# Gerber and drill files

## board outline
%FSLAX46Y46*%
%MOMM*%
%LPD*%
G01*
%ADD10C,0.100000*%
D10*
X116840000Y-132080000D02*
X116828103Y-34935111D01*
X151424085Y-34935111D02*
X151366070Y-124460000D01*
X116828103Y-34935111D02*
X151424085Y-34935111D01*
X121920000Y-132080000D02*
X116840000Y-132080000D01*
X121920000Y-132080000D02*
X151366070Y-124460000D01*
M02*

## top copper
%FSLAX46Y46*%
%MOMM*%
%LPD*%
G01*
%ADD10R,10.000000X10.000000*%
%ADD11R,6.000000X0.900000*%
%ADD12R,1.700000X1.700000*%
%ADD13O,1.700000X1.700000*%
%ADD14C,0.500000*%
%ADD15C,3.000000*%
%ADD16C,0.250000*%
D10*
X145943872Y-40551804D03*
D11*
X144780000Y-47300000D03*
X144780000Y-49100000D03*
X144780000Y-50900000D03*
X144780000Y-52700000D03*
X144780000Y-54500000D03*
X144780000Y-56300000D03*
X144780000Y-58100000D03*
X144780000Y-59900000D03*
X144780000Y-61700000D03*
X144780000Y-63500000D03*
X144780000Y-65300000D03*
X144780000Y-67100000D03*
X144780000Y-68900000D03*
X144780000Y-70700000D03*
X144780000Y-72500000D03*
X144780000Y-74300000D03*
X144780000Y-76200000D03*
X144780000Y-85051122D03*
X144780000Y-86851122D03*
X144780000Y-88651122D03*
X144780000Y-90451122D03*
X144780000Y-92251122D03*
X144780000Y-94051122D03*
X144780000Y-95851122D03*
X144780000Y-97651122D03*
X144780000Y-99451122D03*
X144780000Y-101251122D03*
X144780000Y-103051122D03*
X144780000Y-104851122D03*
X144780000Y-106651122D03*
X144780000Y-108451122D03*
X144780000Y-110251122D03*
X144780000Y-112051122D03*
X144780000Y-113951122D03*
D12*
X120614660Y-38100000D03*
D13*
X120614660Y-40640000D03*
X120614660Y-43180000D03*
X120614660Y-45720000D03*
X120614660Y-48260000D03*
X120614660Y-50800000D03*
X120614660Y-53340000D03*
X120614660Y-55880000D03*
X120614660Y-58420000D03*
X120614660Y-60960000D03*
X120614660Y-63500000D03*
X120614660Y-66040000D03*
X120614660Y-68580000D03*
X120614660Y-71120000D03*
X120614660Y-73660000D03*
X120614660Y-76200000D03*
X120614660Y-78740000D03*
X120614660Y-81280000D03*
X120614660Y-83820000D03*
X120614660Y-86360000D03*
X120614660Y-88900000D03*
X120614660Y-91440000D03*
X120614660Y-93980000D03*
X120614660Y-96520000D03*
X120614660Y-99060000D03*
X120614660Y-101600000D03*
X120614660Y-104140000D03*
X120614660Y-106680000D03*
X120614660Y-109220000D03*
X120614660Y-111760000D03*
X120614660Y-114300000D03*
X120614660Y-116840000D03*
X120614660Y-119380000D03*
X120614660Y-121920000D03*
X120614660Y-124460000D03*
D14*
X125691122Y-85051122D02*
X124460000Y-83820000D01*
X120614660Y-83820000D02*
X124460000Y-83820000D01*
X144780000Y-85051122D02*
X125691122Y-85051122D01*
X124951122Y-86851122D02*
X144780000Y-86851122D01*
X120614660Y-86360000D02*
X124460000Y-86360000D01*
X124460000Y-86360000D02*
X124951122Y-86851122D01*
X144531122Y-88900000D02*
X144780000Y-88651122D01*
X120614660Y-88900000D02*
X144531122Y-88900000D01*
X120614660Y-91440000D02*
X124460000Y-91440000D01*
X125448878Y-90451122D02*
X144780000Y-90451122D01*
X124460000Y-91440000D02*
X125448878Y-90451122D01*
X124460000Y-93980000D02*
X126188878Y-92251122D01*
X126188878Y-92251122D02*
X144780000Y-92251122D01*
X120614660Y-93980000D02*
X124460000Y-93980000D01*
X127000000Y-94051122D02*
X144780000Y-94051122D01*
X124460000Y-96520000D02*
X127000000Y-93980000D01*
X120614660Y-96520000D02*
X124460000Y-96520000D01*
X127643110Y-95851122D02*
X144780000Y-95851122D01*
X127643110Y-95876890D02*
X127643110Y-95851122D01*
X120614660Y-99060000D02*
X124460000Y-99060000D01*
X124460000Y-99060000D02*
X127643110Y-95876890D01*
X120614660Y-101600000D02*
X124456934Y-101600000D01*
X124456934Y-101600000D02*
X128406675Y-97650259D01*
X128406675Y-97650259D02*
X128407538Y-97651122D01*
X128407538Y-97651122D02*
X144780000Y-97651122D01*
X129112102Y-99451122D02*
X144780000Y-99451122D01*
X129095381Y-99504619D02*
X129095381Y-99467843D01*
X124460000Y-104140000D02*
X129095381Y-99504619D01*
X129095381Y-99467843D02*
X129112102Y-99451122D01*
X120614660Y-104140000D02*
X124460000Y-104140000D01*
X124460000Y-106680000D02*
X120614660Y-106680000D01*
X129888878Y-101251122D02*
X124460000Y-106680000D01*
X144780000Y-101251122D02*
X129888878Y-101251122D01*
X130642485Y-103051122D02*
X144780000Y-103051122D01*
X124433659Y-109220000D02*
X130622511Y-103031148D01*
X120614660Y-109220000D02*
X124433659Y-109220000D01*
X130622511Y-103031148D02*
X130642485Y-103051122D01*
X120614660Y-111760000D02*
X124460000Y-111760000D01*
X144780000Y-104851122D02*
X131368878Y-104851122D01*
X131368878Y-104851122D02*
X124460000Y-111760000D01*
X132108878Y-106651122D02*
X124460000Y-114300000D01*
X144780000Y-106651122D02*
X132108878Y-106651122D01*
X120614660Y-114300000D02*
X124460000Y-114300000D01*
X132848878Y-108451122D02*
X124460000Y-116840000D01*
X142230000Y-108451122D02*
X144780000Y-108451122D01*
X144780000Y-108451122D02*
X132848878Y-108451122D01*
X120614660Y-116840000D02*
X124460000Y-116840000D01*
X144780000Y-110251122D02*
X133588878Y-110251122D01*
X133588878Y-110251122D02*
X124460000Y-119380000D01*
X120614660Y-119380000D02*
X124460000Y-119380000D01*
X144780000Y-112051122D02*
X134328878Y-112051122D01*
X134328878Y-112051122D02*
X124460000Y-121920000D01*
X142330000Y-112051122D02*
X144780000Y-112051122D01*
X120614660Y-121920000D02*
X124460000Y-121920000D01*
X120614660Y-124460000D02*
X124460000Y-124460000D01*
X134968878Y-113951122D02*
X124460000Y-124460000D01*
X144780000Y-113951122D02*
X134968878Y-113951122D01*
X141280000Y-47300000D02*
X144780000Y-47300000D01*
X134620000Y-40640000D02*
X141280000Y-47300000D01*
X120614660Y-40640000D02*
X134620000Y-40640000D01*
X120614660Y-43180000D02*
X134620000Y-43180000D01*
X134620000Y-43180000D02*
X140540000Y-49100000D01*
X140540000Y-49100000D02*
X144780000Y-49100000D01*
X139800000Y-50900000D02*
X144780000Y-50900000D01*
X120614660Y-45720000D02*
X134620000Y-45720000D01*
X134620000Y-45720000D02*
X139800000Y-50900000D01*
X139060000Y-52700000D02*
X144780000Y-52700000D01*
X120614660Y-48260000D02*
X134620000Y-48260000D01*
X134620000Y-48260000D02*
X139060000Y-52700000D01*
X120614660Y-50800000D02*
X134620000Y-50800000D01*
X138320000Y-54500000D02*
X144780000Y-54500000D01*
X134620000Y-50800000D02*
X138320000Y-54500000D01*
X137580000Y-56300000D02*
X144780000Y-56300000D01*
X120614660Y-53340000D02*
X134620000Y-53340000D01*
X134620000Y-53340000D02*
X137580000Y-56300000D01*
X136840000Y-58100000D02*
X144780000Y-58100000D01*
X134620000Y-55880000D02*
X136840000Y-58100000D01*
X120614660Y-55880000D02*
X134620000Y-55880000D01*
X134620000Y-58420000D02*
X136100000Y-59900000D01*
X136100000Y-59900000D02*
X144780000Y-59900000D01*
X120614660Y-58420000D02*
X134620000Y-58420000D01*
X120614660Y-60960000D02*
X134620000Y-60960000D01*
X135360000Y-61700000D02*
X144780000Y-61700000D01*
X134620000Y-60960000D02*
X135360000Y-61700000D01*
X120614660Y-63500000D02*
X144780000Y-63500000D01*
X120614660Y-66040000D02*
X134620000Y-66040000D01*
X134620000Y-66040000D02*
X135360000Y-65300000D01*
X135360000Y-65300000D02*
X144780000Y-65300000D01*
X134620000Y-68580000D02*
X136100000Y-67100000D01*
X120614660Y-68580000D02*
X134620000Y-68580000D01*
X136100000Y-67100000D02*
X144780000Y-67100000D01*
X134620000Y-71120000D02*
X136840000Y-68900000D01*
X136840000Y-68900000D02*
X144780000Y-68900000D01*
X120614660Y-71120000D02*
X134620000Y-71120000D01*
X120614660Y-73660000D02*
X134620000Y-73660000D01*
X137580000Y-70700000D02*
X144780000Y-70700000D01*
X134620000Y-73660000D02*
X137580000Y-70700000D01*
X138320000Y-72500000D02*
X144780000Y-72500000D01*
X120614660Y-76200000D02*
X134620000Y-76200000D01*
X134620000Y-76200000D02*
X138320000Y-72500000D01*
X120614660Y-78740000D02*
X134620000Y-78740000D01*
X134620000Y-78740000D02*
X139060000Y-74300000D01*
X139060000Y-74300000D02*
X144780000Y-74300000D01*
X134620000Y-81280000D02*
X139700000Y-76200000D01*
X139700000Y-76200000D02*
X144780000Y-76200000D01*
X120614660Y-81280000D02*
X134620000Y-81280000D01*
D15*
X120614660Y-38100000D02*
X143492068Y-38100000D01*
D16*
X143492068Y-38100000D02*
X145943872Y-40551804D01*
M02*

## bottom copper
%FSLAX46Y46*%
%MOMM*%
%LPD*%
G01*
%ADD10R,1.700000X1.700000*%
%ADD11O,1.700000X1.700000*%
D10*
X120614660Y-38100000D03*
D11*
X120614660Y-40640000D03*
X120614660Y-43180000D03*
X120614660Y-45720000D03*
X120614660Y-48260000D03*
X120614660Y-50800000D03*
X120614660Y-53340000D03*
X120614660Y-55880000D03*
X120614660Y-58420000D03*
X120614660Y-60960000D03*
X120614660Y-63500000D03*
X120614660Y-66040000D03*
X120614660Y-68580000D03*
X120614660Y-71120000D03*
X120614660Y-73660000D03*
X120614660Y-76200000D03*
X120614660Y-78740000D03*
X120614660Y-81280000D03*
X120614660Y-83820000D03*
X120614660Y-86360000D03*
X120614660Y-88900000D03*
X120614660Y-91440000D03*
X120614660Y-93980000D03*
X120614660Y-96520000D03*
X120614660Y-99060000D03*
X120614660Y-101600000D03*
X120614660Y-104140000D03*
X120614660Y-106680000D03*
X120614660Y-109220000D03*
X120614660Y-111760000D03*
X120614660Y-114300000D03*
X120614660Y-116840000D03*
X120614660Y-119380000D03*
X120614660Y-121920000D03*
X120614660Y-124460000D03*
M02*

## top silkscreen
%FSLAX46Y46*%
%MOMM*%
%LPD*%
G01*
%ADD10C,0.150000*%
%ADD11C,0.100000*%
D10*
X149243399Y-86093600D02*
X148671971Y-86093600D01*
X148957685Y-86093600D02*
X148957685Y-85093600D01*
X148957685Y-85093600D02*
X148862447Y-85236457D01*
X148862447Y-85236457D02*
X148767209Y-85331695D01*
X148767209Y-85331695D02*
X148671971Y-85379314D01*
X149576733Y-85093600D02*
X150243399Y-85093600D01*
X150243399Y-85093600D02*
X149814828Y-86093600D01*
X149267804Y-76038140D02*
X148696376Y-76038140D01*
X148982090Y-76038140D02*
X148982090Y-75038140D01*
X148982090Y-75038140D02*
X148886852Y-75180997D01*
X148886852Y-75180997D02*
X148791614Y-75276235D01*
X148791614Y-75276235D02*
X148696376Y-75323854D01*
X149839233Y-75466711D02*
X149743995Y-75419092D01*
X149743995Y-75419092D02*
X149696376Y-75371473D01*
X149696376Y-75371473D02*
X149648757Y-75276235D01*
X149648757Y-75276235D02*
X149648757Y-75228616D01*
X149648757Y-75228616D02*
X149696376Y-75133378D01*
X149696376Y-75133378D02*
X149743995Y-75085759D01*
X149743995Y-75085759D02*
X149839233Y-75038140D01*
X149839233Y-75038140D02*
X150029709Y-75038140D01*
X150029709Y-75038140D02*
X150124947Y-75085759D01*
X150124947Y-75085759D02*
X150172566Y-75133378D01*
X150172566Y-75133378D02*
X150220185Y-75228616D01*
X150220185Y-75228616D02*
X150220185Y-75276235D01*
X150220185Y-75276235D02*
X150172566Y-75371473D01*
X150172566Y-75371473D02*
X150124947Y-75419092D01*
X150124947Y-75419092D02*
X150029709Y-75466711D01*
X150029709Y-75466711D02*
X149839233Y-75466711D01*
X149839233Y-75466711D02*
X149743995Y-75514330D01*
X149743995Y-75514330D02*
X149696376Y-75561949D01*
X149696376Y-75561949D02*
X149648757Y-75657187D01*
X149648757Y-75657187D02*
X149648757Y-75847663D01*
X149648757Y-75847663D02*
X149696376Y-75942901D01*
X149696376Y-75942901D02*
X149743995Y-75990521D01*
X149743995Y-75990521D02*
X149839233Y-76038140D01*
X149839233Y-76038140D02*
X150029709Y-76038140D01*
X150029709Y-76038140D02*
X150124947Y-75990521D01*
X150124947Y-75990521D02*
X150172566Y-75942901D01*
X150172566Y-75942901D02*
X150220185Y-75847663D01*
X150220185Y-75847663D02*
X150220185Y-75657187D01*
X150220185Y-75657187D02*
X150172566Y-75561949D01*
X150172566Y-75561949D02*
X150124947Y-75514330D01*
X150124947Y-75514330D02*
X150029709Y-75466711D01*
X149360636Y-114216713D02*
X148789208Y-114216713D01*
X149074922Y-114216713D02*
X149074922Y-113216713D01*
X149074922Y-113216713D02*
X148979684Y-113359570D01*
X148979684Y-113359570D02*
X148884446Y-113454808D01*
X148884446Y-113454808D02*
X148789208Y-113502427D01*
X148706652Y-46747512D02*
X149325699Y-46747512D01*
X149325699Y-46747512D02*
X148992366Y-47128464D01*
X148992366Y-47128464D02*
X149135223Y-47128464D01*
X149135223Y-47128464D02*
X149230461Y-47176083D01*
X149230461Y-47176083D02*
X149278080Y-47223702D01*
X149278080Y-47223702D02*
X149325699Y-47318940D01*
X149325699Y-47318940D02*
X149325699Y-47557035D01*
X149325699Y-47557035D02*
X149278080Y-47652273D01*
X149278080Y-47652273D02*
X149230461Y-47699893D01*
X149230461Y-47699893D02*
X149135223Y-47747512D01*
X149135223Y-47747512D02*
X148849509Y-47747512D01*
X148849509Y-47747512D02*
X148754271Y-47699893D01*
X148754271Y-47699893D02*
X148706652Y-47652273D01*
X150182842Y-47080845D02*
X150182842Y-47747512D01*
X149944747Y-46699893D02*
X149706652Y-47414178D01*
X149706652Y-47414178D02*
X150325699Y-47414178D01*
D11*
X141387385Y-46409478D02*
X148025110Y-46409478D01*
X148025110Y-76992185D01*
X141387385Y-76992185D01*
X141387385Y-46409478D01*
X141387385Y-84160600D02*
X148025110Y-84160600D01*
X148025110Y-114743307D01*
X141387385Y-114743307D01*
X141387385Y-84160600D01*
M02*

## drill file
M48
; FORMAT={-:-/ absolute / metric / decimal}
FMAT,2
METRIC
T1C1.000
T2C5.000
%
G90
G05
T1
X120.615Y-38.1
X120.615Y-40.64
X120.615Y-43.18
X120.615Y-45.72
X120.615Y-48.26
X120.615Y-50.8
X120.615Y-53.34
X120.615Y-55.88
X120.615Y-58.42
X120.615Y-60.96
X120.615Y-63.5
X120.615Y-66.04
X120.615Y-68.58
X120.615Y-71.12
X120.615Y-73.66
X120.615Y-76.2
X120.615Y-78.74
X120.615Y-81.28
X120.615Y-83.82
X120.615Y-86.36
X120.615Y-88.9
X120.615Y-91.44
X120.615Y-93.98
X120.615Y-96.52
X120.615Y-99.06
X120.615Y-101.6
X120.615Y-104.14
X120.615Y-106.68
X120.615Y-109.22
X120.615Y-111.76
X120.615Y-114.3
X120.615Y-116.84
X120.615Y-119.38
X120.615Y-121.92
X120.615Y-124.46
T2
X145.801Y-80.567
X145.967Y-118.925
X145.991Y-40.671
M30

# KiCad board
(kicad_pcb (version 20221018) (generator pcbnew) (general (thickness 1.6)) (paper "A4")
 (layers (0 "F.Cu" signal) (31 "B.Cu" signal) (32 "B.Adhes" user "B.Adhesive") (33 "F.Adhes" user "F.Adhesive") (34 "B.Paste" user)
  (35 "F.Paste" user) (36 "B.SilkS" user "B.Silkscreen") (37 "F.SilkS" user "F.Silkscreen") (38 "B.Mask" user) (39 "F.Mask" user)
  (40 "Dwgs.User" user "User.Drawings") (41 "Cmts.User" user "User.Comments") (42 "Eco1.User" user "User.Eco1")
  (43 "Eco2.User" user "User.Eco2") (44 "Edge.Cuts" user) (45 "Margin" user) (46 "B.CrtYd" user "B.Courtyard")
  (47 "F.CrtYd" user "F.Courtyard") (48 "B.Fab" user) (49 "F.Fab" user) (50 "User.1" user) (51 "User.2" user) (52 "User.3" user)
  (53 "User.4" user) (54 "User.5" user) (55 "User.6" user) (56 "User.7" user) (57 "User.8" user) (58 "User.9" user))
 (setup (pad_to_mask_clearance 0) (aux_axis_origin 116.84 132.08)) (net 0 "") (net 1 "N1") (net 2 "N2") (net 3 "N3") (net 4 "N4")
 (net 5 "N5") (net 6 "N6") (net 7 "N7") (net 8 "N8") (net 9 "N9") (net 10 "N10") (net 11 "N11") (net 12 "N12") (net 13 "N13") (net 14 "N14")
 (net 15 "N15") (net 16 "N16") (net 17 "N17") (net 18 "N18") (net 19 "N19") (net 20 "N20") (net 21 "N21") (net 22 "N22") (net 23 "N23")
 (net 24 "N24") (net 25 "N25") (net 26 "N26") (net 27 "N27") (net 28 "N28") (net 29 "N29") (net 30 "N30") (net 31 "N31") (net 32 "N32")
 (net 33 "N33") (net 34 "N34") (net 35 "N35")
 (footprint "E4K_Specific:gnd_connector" (layer "F.Cu") (at 145.943872 41.551804)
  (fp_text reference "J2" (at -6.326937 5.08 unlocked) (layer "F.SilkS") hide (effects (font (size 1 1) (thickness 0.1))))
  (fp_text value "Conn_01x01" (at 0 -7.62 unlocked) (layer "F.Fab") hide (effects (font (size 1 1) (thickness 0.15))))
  (pad "1" smd rect (at 0 -1) (size 10 10) (layers "F.Cu" "F.Mask") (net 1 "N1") (thermal_bridge_angle 45)))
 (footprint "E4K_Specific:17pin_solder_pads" (layer "F.Cu") (at 140.90939 77.748878)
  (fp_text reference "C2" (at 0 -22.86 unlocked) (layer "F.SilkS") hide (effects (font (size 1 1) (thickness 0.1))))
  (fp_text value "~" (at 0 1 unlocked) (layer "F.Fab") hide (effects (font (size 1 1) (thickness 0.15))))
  (fp_rect (start 0.477995 -31.3394) (end 7.11572 -0.756693) (stroke (width 0.1) (type solid)) (fill none) (layer "F.SilkS"))
  (pad "1" smd rect (at 3.87061 -30.448878) (size 6 0.9) (layers "F.Cu" "F.Mask") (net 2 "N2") (thermal_bridge_angle 45))
  (pad "2" smd rect (at 3.87061 -28.648878) (size 6 0.9) (layers "F.Cu" "F.Mask") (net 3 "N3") (thermal_bridge_angle 45))
  (pad "3" smd rect (at 3.87061 -26.848878) (size 6 0.9) (layers "F.Cu" "F.Mask") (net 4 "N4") (thermal_bridge_angle 45))
  (pad "4" smd rect (at 3.87061 -25.048878) (size 6 0.9) (layers "F.Cu" "F.Mask") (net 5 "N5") (thermal_bridge_angle 45))
  (pad "5" smd rect (at 3.87061 -23.248878) (size 6 0.9) (layers "F.Cu" "F.Mask") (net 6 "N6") (thermal_bridge_angle 45))
  (pad "6" smd rect (at 3.87061 -21.448878) (size 6 0.9) (layers "F.Cu" "F.Mask") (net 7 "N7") (thermal_bridge_angle 45))
  (pad "7" smd rect (at 3.87061 -19.648878) (size 6 0.9) (layers "F.Cu" "F.Mask") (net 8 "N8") (thermal_bridge_angle 45))
  (pad "8" smd rect (at 3.87061 -17.848878) (size 6 0.9) (layers "F.Cu" "F.Mask") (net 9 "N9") (thermal_bridge_angle 45))
  (pad "9" smd rect (at 3.87061 -16.048878) (size 6 0.9) (layers "F.Cu" "F.Mask") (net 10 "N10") (thermal_bridge_angle 45))
  (pad "10" smd rect (at 3.87061 -14.248878) (size 6 0.9) (layers "F.Cu" "F.Mask") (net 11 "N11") (thermal_bridge_angle 45))
  (pad "11" smd rect (at 3.87061 -12.448878) (size 6 0.9) (layers "F.Cu" "F.Mask") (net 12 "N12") (thermal_bridge_angle 45))
  (pad "12" smd rect (at 3.87061 -10.648878) (size 6 0.9) (layers "F.Cu" "F.Mask") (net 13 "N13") (thermal_bridge_angle 45))
  (pad "13" smd rect (at 3.87061 -8.848878) (size 6 0.9) (layers "F.Cu" "F.Mask") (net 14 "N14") (thermal_bridge_angle 45))
  (pad "14" smd rect (at 3.87061 -7.048878) (size 6 0.9) (layers "F.Cu" "F.Mask") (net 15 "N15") (thermal_bridge_angle 45))
  (pad "15" smd rect (at 3.87061 -5.248878) (size 6 0.9) (layers "F.Cu" "F.Mask") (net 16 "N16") (thermal_bridge_angle 45))
  (pad "16" smd rect (at 3.87061 -3.448878) (size 6 0.9) (layers "F.Cu" "F.Mask") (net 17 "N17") (thermal_bridge_angle 45))
  (pad "17" smd rect (at 3.87061 -1.548878) (size 6 0.9) (layers "F.Cu" "F.Mask") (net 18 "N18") (thermal_bridge_angle 45)))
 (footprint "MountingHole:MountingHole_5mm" (layer "F.Cu") (at 145.966762 118.924527)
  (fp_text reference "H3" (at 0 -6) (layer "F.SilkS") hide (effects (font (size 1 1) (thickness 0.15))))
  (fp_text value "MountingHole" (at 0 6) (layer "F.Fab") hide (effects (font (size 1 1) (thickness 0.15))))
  (pad "" np_thru_hole circle (at 0 0) (size 5 5) (drill 5) (layers "*.Cu" "*.Mask")))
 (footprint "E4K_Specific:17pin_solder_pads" (layer "F.Cu") (at 140.90939 115.5)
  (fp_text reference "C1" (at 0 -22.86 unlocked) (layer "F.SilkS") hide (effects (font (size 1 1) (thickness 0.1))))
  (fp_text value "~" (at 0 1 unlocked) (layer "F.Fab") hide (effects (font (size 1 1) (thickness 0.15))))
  (fp_rect (start 0.477995 -31.3394) (end 7.11572 -0.756693) (stroke (width 0.1) (type solid)) (fill none) (layer "F.SilkS"))
  (pad "1" smd rect (at 3.87061 -30.448878) (size 6 0.9) (layers "F.Cu" "F.Mask") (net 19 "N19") (thermal_bridge_angle 45))
  (pad "2" smd rect (at 3.87061 -28.648878) (size 6 0.9) (layers "F.Cu" "F.Mask") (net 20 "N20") (thermal_bridge_angle 45))
  (pad "3" smd rect (at 3.87061 -26.848878) (size 6 0.9) (layers "F.Cu" "F.Mask") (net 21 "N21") (thermal_bridge_angle 45))
  (pad "4" smd rect (at 3.87061 -25.048878) (size 6 0.9) (layers "F.Cu" "F.Mask") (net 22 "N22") (thermal_bridge_angle 45))
  (pad "5" smd rect (at 3.87061 -23.248878) (size 6 0.9) (layers "F.Cu" "F.Mask") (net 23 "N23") (thermal_bridge_angle 45))
  (pad "6" smd rect (at 3.87061 -21.448878) (size 6 0.9) (layers "F.Cu" "F.Mask") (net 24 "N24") (thermal_bridge_angle 45))
  (pad "7" smd rect (at 3.87061 -19.648878) (size 6 0.9) (layers "F.Cu" "F.Mask") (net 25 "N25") (thermal_bridge_angle 45))
  (pad "8" smd rect (at 3.87061 -17.848878) (size 6 0.9) (layers "F.Cu" "F.Mask") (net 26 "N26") (thermal_bridge_angle 45))
  (pad "9" smd rect (at 3.87061 -16.048878) (size 6 0.9) (layers "F.Cu" "F.Mask") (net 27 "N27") (thermal_bridge_angle 45))
  (pad "10" smd rect (at 3.87061 -14.248878) (size 6 0.9) (layers "F.Cu" "F.Mask") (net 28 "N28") (thermal_bridge_angle 45))
  (pad "11" smd rect (at 3.87061 -12.448878) (size 6 0.9) (layers "F.Cu" "F.Mask") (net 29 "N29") (thermal_bridge_angle 45))
  (pad "12" smd rect (at 3.87061 -10.648878) (size 6 0.9) (layers "F.Cu" "F.Mask") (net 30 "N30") (thermal_bridge_angle 45))
  (pad "13" smd rect (at 3.87061 -8.848878) (size 6 0.9) (layers "F.Cu" "F.Mask") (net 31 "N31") (thermal_bridge_angle 45))
  (pad "14" smd rect (at 3.87061 -7.048878) (size 6 0.9) (layers "F.Cu" "F.Mask") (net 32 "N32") (thermal_bridge_angle 45))
  (pad "15" smd rect (at 3.87061 -5.248878) (size 6 0.9) (layers "F.Cu" "F.Mask") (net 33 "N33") (thermal_bridge_angle 45))
  (pad "16" smd rect (at 3.87061 -3.448878) (size 6 0.9) (layers "F.Cu" "F.Mask") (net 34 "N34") (thermal_bridge_angle 45))
  (pad "17" smd rect (at 3.87061 -1.548878) (size 6 0.9) (layers "F.Cu" "F.Mask") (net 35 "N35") (thermal_bridge_angle 45)))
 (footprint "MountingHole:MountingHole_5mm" (layer "F.Cu") (at 145.801463 80.567457)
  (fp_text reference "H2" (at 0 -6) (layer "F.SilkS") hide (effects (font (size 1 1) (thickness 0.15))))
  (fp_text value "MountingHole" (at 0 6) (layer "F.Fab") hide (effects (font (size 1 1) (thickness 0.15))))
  (pad "" np_thru_hole circle (at 0 0) (size 5 5) (drill 5) (layers "*.Cu" "*.Mask")))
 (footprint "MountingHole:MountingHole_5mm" (layer "F.Cu") (at 145.99109 40.671151)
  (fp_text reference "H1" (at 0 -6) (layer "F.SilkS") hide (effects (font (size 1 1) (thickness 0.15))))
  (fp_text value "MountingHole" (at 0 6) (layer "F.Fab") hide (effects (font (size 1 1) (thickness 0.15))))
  (pad "" np_thru_hole circle (at 0 0) (size 5 5) (drill 5) (layers "*.Cu" "*.Mask")))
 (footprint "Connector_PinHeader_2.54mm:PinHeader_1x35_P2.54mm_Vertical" (layer "B.Cu") (at 120.61466 38.1 180)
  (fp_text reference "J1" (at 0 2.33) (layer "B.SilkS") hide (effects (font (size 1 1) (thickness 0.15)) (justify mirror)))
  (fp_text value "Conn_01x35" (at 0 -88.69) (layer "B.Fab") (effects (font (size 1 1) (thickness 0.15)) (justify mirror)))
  (pad "1" thru_hole rect (at 0 0 180) (size 1.7 1.7) (drill 1) (layers "*.Cu" "*.Mask") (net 1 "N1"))
  (pad "2" thru_hole oval (at 0 -2.54 180) (size 1.7 1.7) (drill 1) (layers "*.Cu" "*.Mask") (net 2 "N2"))
  (pad "3" thru_hole oval (at 0 -5.08 180) (size 1.7 1.7) (drill 1) (layers "*.Cu" "*.Mask") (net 3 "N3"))
  (pad "4" thru_hole oval (at 0 -7.62 180) (size 1.7 1.7) (drill 1) (layers "*.Cu" "*.Mask") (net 4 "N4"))
  (pad "5" thru_hole oval (at 0 -10.16 180) (size 1.7 1.7) (drill 1) (layers "*.Cu" "*.Mask") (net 5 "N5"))
  (pad "6" thru_hole oval (at 0 -12.7 180) (size 1.7 1.7) (drill 1) (layers "*.Cu" "*.Mask") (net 6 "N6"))
  (pad "7" thru_hole oval (at 0 -15.24 180) (size 1.7 1.7) (drill 1) (layers "*.Cu" "*.Mask") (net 7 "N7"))
  (pad "8" thru_hole oval (at 0 -17.78 180) (size 1.7 1.7) (drill 1) (layers "*.Cu" "*.Mask") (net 8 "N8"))
  (pad "9" thru_hole oval (at 0 -20.32 180) (size 1.7 1.7) (drill 1) (layers "*.Cu" "*.Mask") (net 9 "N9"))
  (pad "10" thru_hole oval (at 0 -22.86 180) (size 1.7 1.7) (drill 1) (layers "*.Cu" "*.Mask") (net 10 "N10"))
  (pad "11" thru_hole oval (at 0 -25.4 180) (size 1.7 1.7) (drill 1) (layers "*.Cu" "*.Mask") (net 11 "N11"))
  (pad "12" thru_hole oval (at 0 -27.94 180) (size 1.7 1.7) (drill 1) (layers "*.Cu" "*.Mask") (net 12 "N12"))
  (pad "13" thru_hole oval (at 0 -30.48 180) (size 1.7 1.7) (drill 1) (layers "*.Cu" "*.Mask") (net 13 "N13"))
  (pad "14" thru_hole oval (at 0 -33.02 180) (size 1.7 1.7) (drill 1) (layers "*.Cu" "*.Mask") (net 14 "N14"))
  (pad "15" thru_hole oval (at 0 -35.56 180) (size 1.7 1.7) (drill 1) (layers "*.Cu" "*.Mask") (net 15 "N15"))
  (pad "16" thru_hole oval (at 0 -38.1 180) (size 1.7 1.7) (drill 1) (layers "*.Cu" "*.Mask") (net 16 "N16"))
  (pad "17" thru_hole oval (at 0 -40.64 180) (size 1.7 1.7) (drill 1) (layers "*.Cu" "*.Mask") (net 17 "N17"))
  (pad "18" thru_hole oval (at 0 -43.18 180) (size 1.7 1.7) (drill 1) (layers "*.Cu" "*.Mask") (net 18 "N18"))
  (pad "19" thru_hole oval (at 0 -45.72 180) (size 1.7 1.7) (drill 1) (layers "*.Cu" "*.Mask") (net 19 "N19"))
  (pad "20" thru_hole oval (at 0 -48.26 180) (size 1.7 1.7) (drill 1) (layers "*.Cu" "*.Mask") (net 20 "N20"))
  (pad "21" thru_hole oval (at 0 -50.8 180) (size 1.7 1.7) (drill 1) (layers "*.Cu" "*.Mask") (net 21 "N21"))
  (pad "22" thru_hole oval (at 0 -53.34 180) (size 1.7 1.7) (drill 1) (layers "*.Cu" "*.Mask") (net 22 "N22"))
  (pad "23" thru_hole oval (at 0 -55.88 180) (size 1.7 1.7) (drill 1) (layers "*.Cu" "*.Mask") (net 23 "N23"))
  (pad "24" thru_hole oval (at 0 -58.42 180) (size 1.7 1.7) (drill 1) (layers "*.Cu" "*.Mask") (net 24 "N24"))
  (pad "25" thru_hole oval (at 0 -60.96 180) (size 1.7 1.7) (drill 1) (layers "*.Cu" "*.Mask") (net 25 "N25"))
  (pad "26" thru_hole oval (at 0 -63.5 180) (size 1.7 1.7) (drill 1) (layers "*.Cu" "*.Mask") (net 26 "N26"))
  (pad "27" thru_hole oval (at 0 -66.04 180) (size 1.7 1.7) (drill 1) (layers "*.Cu" "*.Mask") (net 27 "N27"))
  (pad "28" thru_hole oval (at 0 -68.58 180) (size 1.7 1.7) (drill 1) (layers "*.Cu" "*.Mask") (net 28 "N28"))
  (pad "29" thru_hole oval (at 0 -71.12 180) (size 1.7 1.7) (drill 1) (layers "*.Cu" "*.Mask") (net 29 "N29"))
  (pad "30" thru_hole oval (at 0 -73.66 180) (size 1.7 1.7) (drill 1) (layers "*.Cu" "*.Mask") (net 30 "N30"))
  (pad "31" thru_hole oval (at 0 -76.2 180) (size 1.7 1.7) (drill 1) (layers "*.Cu" "*.Mask") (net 31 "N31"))
  (pad "32" thru_hole oval (at 0 -78.74 180) (size 1.7 1.7) (drill 1) (layers "*.Cu" "*.Mask") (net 32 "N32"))
  (pad "33" thru_hole oval (at 0 -81.28 180) (size 1.7 1.7) (drill 1) (layers "*.Cu" "*.Mask") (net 33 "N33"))
  (pad "34" thru_hole oval (at 0 -83.82 180) (size 1.7 1.7) (drill 1) (layers "*.Cu" "*.Mask") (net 34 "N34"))
  (pad "35" thru_hole oval (at 0 -86.36 180) (size 1.7 1.7) (drill 1) (layers "*.Cu" "*.Mask") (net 35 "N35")))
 (gr_line (start 116.84 132.08) (end 116.828103 34.935111) (stroke (width 0.1) (type default)) (layer "Edge.Cuts"))
 (gr_line (start 151.424085 34.935111) (end 151.36607 124.46) (stroke (width 0.1) (type default)) (layer "Edge.Cuts"))
 (gr_line (start 116.828103 34.935111) (end 151.424085 34.935111) (stroke (width 0.1) (type default)) (layer "Edge.Cuts"))
 (gr_line (start 121.92 132.08) (end 116.84 132.08) (stroke (width 0.1) (type default)) (layer "Edge.Cuts"))
 (gr_line (start 121.92 132.08) (end 151.36607 124.46) (stroke (width 0.1) (type default)) (layer "Edge.Cuts"))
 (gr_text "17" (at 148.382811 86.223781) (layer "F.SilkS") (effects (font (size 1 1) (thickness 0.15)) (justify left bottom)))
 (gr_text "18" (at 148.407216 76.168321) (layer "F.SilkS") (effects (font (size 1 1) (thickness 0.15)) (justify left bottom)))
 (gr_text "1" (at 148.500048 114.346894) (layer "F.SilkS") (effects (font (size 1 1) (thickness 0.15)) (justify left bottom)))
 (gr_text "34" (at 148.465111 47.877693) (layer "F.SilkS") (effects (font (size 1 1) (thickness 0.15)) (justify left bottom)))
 (segment (start 125.691122 85.051122) (end 124.46 83.82) (width 0.5) (layer "F.Cu") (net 19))
 (segment (start 120.61466 83.82) (end 124.46 83.82) (width 0.5) (layer "F.Cu") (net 19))
 (segment (start 144.78 85.051122) (end 125.691122 85.051122) (width 0.5) (layer "F.Cu") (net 19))
 (segment (start 124.951122 86.851122) (end 144.78 86.851122) (width 0.5) (layer "F.Cu") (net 20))
 (segment (start 120.61466 86.36) (end 124.46 86.36) (width 0.5) (layer "F.Cu") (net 20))
 (segment (start 124.46 86.36) (end 124.951122 86.851122) (width 0.5) (layer "F.Cu") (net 20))
 (segment (start 144.531122 88.9) (end 144.78 88.651122) (width 0.5) (layer "F.Cu") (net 21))
 (segment (start 120.61466 88.9) (end 144.531122 88.9) (width 0.5) (layer "F.Cu") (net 21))
 (segment (start 120.61466 91.44) (end 124.46 91.44) (width 0.5) (layer "F.Cu") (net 22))
 (segment (start 125.448878 90.451122) (end 144.78 90.451122) (width 0.5) (layer "F.Cu") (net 22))
 (segment (start 124.46 91.44) (end 125.448878 90.451122) (width 0.5) (layer "F.Cu") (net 22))
 (segment (start 124.46 93.98) (end 126.188878 92.251122) (width 0.5) (layer "F.Cu") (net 23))
 (segment (start 126.188878 92.251122) (end 144.78 92.251122) (width 0.5) (layer "F.Cu") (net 23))
 (segment (start 120.61466 93.98) (end 124.46 93.98) (width 0.5) (layer "F.Cu") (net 23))
 (segment (start 127 94.051122) (end 144.78 94.051122) (width 0.5) (layer "F.Cu") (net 24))
 (segment (start 124.46 96.52) (end 127 93.98) (width 0.5) (layer "F.Cu") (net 24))
 (segment (start 120.61466 96.52) (end 124.46 96.52) (width 0.5) (layer "F.Cu") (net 24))
 (segment (start 127.64311 95.851122) (end 144.78 95.851122) (width 0.5) (layer "F.Cu") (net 25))
 (segment (start 127.64311 95.87689) (end 127.64311 95.851122) (width 0.5) (layer "F.Cu") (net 25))
 (segment (start 120.61466 99.06) (end 124.46 99.06) (width 0.5) (layer "F.Cu") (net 25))
 (segment (start 124.46 99.06) (end 127.64311 95.87689) (width 0.5) (layer "F.Cu") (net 25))
 (segment (start 120.61466 101.6) (end 124.456934 101.6) (width 0.5) (layer "F.Cu") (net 26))
 (segment (start 124.456934 101.6) (end 128.406675 97.650259) (width 0.5) (layer "F.Cu") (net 26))
 (segment (start 128.406675 97.650259) (end 128.407538 97.651122) (width 0.5) (layer "F.Cu") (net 26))
 (segment (start 128.407538 97.651122) (end 144.78 97.651122) (width 0.5) (layer "F.Cu") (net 26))
 (segment (start 129.112102 99.451122) (end 144.78 99.451122) (width 0.5) (layer "F.Cu") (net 27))
 (segment (start 129.095381 99.504619) (end 129.095381 99.467843) (width 0.5) (layer "F.Cu") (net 27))
 (segment (start 124.46 104.14) (end 129.095381 99.504619) (width 0.5) (layer "F.Cu") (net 27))
 (segment (start 129.095381 99.467843) (end 129.112102 99.451122) (width 0.5) (layer "F.Cu") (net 27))
 (segment (start 120.61466 104.14) (end 124.46 104.14) (width 0.5) (layer "F.Cu") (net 27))
 (segment (start 124.46 106.68) (end 120.61466 106.68) (width 0.5) (layer "F.Cu") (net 28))
 (segment (start 129.888878 101.251122) (end 124.46 106.68) (width 0.5) (layer "F.Cu") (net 28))
 (segment (start 144.78 101.251122) (end 129.888878 101.251122) (width 0.5) (layer "F.Cu") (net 28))
 (segment (start 130.642485 103.051122) (end 144.78 103.051122) (width 0.5) (layer "F.Cu") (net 29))
 (segment (start 124.433659 109.22) (end 130.622511 103.031148) (width 0.5) (layer "F.Cu") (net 29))
 (segment (start 120.61466 109.22) (end 124.433659 109.22) (width 0.5) (layer "F.Cu") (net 29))
 (segment (start 130.622511 103.031148) (end 130.642485 103.051122) (width 0.5) (layer "F.Cu") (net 29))
 (segment (start 120.61466 111.76) (end 124.46 111.76) (width 0.5) (layer "F.Cu") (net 30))
 (segment (start 144.78 104.851122) (end 131.368878 104.851122) (width 0.5) (layer "F.Cu") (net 30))
 (segment (start 131.368878 104.851122) (end 124.46 111.76) (width 0.5) (layer "F.Cu") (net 30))
 (segment (start 132.108878 106.651122) (end 124.46 114.3) (width 0.5) (layer "F.Cu") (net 31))
 (segment (start 144.78 106.651122) (end 132.108878 106.651122) (width 0.5) (layer "F.Cu") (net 31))
 (segment (start 120.61466 114.3) (end 124.46 114.3) (width 0.5) (layer "F.Cu") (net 31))
 (segment (start 132.848878 108.451122) (end 124.46 116.84) (width 0.5) (layer "F.Cu") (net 32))
 (segment (start 142.23 108.451122) (end 144.78 108.451122) (width 0.5) (layer "F.Cu") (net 32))
 (segment (start 144.78 108.451122) (end 132.848878 108.451122) (width 0.5) (layer "F.Cu") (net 32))
 (segment (start 120.61466 116.84) (end 124.46 116.84) (width 0.5) (layer "F.Cu") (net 32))
 (segment (start 144.78 110.251122) (end 133.588878 110.251122) (width 0.5) (layer "F.Cu") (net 33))
 (segment (start 133.588878 110.251122) (end 124.46 119.38) (width 0.5) (layer "F.Cu") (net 33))
 (segment (start 120.61466 119.38) (end 124.46 119.38) (width 0.5) (layer "F.Cu") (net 33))
 (segment (start 144.78 112.051122) (end 134.328878 112.051122) (width 0.5) (layer "F.Cu") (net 34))
 (segment (start 134.328878 112.051122) (end 124.46 121.92) (width 0.5) (layer "F.Cu") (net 34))
 (segment (start 142.33 112.051122) (end 144.78 112.051122) (width 0.5) (layer "F.Cu") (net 34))
 (segment (start 120.61466 121.92) (end 124.46 121.92) (width 0.5) (layer "F.Cu") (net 34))
 (segment (start 120.61466 124.46) (end 124.46 124.46) (width 0.5) (layer "F.Cu") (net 35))
 (segment (start 134.968878 113.951122) (end 124.46 124.46) (width 0.5) (layer "F.Cu") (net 35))
 (segment (start 144.78 113.951122) (end 134.968878 113.951122) (width 0.5) (layer "F.Cu") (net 35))
 (segment (start 141.28 47.3) (end 144.78 47.3) (width 0.5) (layer "F.Cu") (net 2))
 (segment (start 134.62 40.64) (end 141.28 47.3) (width 0.5) (layer "F.Cu") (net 2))
 (segment (start 120.61466 40.64) (end 134.62 40.64) (width 0.5) (layer "F.Cu") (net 2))
 (segment (start 120.61466 43.18) (end 134.62 43.18) (width 0.5) (layer "F.Cu") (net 3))
 (segment (start 134.62 43.18) (end 140.54 49.1) (width 0.5) (layer "F.Cu") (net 3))
 (segment (start 140.54 49.1) (end 144.78 49.1) (width 0.5) (layer "F.Cu") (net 3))
 (segment (start 139.8 50.9) (end 144.78 50.9) (width 0.5) (layer "F.Cu") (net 4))
 (segment (start 120.61466 45.72) (end 134.62 45.72) (width 0.5) (layer "F.Cu") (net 4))
 (segment (start 134.62 45.72) (end 139.8 50.9) (width 0.5) (layer "F.Cu") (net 4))
 (segment (start 139.06 52.7) (end 144.78 52.7) (width 0.5) (layer "F.Cu") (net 5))
 (segment (start 120.61466 48.26) (end 134.62 48.26) (width 0.5) (layer "F.Cu") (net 5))
 (segment (start 134.62 48.26) (end 139.06 52.7) (width 0.5) (layer "F.Cu") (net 5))
 (segment (start 120.61466 50.8) (end 134.62 50.8) (width 0.5) (layer "F.Cu") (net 6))
 (segment (start 138.32 54.5) (end 144.78 54.5) (width 0.5) (layer "F.Cu") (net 6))
 (segment (start 134.62 50.8) (end 138.32 54.5) (width 0.5) (layer "F.Cu") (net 6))
 (segment (start 137.58 56.3) (end 144.78 56.3) (width 0.5) (layer "F.Cu") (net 7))
 (segment (start 120.61466 53.34) (end 134.62 53.34) (width 0.5) (layer "F.Cu") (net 7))
 (segment (start 134.62 53.34) (end 137.58 56.3) (width 0.5) (layer "F.Cu") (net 7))
 (segment (start 136.84 58.1) (end 144.78 58.1) (width 0.5) (layer "F.Cu") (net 8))
 (segment (start 134.62 55.88) (end 136.84 58.1) (width 0.5) (layer "F.Cu") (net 8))
 (segment (start 120.61466 55.88) (end 134.62 55.88) (width 0.5) (layer "F.Cu") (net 8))
 (segment (start 134.62 58.42) (end 136.1 59.9) (width 0.5) (layer "F.Cu") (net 9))
 (segment (start 136.1 59.9) (end 144.78 59.9) (width 0.5) (layer "F.Cu") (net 9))
 (segment (start 120.61466 58.42) (end 134.62 58.42) (width 0.5) (layer "F.Cu") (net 9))
 (segment (start 120.61466 60.96) (end 134.62 60.96) (width 0.5) (layer "F.Cu") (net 10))
 (segment (start 135.36 61.7) (end 144.78 61.7) (width 0.5) (layer "F.Cu") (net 10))
 (segment (start 134.62 60.96) (end 135.36 61.7) (width 0.5) (layer "F.Cu") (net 10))
 (segment (start 120.61466 63.5) (end 144.78 63.5) (width 0.5) (layer "F.Cu") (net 11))
 (segment (start 120.61466 66.04) (end 134.62 66.04) (width 0.5) (layer "F.Cu") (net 12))
 (segment (start 134.62 66.04) (end 135.36 65.3) (width 0.5) (layer "F.Cu") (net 12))
 (segment (start 135.36 65.3) (end 144.78 65.3) (width 0.5) (layer "F.Cu") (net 12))
 (segment (start 134.62 68.58) (end 136.1 67.1) (width 0.5) (layer "F.Cu") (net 13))
 (segment (start 120.61466 68.58) (end 134.62 68.58) (width 0.5) (layer "F.Cu") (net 13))
 (segment (start 136.1 67.1) (end 144.78 67.1) (width 0.5) (layer "F.Cu") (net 13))
 (segment (start 134.62 71.12) (end 136.84 68.9) (width 0.5) (layer "F.Cu") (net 14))
 (segment (start 136.84 68.9) (end 144.78 68.9) (width 0.5) (layer "F.Cu") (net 14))
 (segment (start 120.61466 71.12) (end 134.62 71.12) (width 0.5) (layer "F.Cu") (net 14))
 (segment (start 120.61466 73.66) (end 134.62 73.66) (width 0.5) (layer "F.Cu") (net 15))
 (segment (start 137.58 70.7) (end 144.78 70.7) (width 0.5) (layer "F.Cu") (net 15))
 (segment (start 134.62 73.66) (end 137.58 70.7) (width 0.5) (layer "F.Cu") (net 15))
 (segment (start 138.32 72.5) (end 144.78 72.5) (width 0.5) (layer "F.Cu") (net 16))
 (segment (start 120.61466 76.2) (end 134.62 76.2) (width 0.5) (layer "F.Cu") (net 16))
 (segment (start 134.62 76.2) (end 138.32 72.5) (width 0.5) (layer "F.Cu") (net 16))
 (segment (start 120.61466 78.74) (end 134.62 78.74) (width 0.5) (layer "F.Cu") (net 17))
 (segment (start 134.62 78.74) (end 139.06 74.3) (width 0.5) (layer "F.Cu") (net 17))
 (segment (start 139.06 74.3) (end 144.78 74.3) (width 0.5) (layer "F.Cu") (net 17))
 (segment (start 134.62 81.28) (end 139.7 76.2) (width 0.5) (layer "F.Cu") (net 18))
 (segment (start 139.7 76.2) (end 144.78 76.2) (width 0.5) (layer "F.Cu") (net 18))
 (segment (start 120.61466 81.28) (end 134.62 81.28) (width 0.5) (layer "F.Cu") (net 18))
 (segment (start 120.61466 38.1) (end 143.492068 38.1) (width 3) (layer "F.Cu") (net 1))
 (segment (start 143.492068 38.1) (end 145.943872 40.551804) (width 0.25) (layer "F.Cu") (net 1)))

